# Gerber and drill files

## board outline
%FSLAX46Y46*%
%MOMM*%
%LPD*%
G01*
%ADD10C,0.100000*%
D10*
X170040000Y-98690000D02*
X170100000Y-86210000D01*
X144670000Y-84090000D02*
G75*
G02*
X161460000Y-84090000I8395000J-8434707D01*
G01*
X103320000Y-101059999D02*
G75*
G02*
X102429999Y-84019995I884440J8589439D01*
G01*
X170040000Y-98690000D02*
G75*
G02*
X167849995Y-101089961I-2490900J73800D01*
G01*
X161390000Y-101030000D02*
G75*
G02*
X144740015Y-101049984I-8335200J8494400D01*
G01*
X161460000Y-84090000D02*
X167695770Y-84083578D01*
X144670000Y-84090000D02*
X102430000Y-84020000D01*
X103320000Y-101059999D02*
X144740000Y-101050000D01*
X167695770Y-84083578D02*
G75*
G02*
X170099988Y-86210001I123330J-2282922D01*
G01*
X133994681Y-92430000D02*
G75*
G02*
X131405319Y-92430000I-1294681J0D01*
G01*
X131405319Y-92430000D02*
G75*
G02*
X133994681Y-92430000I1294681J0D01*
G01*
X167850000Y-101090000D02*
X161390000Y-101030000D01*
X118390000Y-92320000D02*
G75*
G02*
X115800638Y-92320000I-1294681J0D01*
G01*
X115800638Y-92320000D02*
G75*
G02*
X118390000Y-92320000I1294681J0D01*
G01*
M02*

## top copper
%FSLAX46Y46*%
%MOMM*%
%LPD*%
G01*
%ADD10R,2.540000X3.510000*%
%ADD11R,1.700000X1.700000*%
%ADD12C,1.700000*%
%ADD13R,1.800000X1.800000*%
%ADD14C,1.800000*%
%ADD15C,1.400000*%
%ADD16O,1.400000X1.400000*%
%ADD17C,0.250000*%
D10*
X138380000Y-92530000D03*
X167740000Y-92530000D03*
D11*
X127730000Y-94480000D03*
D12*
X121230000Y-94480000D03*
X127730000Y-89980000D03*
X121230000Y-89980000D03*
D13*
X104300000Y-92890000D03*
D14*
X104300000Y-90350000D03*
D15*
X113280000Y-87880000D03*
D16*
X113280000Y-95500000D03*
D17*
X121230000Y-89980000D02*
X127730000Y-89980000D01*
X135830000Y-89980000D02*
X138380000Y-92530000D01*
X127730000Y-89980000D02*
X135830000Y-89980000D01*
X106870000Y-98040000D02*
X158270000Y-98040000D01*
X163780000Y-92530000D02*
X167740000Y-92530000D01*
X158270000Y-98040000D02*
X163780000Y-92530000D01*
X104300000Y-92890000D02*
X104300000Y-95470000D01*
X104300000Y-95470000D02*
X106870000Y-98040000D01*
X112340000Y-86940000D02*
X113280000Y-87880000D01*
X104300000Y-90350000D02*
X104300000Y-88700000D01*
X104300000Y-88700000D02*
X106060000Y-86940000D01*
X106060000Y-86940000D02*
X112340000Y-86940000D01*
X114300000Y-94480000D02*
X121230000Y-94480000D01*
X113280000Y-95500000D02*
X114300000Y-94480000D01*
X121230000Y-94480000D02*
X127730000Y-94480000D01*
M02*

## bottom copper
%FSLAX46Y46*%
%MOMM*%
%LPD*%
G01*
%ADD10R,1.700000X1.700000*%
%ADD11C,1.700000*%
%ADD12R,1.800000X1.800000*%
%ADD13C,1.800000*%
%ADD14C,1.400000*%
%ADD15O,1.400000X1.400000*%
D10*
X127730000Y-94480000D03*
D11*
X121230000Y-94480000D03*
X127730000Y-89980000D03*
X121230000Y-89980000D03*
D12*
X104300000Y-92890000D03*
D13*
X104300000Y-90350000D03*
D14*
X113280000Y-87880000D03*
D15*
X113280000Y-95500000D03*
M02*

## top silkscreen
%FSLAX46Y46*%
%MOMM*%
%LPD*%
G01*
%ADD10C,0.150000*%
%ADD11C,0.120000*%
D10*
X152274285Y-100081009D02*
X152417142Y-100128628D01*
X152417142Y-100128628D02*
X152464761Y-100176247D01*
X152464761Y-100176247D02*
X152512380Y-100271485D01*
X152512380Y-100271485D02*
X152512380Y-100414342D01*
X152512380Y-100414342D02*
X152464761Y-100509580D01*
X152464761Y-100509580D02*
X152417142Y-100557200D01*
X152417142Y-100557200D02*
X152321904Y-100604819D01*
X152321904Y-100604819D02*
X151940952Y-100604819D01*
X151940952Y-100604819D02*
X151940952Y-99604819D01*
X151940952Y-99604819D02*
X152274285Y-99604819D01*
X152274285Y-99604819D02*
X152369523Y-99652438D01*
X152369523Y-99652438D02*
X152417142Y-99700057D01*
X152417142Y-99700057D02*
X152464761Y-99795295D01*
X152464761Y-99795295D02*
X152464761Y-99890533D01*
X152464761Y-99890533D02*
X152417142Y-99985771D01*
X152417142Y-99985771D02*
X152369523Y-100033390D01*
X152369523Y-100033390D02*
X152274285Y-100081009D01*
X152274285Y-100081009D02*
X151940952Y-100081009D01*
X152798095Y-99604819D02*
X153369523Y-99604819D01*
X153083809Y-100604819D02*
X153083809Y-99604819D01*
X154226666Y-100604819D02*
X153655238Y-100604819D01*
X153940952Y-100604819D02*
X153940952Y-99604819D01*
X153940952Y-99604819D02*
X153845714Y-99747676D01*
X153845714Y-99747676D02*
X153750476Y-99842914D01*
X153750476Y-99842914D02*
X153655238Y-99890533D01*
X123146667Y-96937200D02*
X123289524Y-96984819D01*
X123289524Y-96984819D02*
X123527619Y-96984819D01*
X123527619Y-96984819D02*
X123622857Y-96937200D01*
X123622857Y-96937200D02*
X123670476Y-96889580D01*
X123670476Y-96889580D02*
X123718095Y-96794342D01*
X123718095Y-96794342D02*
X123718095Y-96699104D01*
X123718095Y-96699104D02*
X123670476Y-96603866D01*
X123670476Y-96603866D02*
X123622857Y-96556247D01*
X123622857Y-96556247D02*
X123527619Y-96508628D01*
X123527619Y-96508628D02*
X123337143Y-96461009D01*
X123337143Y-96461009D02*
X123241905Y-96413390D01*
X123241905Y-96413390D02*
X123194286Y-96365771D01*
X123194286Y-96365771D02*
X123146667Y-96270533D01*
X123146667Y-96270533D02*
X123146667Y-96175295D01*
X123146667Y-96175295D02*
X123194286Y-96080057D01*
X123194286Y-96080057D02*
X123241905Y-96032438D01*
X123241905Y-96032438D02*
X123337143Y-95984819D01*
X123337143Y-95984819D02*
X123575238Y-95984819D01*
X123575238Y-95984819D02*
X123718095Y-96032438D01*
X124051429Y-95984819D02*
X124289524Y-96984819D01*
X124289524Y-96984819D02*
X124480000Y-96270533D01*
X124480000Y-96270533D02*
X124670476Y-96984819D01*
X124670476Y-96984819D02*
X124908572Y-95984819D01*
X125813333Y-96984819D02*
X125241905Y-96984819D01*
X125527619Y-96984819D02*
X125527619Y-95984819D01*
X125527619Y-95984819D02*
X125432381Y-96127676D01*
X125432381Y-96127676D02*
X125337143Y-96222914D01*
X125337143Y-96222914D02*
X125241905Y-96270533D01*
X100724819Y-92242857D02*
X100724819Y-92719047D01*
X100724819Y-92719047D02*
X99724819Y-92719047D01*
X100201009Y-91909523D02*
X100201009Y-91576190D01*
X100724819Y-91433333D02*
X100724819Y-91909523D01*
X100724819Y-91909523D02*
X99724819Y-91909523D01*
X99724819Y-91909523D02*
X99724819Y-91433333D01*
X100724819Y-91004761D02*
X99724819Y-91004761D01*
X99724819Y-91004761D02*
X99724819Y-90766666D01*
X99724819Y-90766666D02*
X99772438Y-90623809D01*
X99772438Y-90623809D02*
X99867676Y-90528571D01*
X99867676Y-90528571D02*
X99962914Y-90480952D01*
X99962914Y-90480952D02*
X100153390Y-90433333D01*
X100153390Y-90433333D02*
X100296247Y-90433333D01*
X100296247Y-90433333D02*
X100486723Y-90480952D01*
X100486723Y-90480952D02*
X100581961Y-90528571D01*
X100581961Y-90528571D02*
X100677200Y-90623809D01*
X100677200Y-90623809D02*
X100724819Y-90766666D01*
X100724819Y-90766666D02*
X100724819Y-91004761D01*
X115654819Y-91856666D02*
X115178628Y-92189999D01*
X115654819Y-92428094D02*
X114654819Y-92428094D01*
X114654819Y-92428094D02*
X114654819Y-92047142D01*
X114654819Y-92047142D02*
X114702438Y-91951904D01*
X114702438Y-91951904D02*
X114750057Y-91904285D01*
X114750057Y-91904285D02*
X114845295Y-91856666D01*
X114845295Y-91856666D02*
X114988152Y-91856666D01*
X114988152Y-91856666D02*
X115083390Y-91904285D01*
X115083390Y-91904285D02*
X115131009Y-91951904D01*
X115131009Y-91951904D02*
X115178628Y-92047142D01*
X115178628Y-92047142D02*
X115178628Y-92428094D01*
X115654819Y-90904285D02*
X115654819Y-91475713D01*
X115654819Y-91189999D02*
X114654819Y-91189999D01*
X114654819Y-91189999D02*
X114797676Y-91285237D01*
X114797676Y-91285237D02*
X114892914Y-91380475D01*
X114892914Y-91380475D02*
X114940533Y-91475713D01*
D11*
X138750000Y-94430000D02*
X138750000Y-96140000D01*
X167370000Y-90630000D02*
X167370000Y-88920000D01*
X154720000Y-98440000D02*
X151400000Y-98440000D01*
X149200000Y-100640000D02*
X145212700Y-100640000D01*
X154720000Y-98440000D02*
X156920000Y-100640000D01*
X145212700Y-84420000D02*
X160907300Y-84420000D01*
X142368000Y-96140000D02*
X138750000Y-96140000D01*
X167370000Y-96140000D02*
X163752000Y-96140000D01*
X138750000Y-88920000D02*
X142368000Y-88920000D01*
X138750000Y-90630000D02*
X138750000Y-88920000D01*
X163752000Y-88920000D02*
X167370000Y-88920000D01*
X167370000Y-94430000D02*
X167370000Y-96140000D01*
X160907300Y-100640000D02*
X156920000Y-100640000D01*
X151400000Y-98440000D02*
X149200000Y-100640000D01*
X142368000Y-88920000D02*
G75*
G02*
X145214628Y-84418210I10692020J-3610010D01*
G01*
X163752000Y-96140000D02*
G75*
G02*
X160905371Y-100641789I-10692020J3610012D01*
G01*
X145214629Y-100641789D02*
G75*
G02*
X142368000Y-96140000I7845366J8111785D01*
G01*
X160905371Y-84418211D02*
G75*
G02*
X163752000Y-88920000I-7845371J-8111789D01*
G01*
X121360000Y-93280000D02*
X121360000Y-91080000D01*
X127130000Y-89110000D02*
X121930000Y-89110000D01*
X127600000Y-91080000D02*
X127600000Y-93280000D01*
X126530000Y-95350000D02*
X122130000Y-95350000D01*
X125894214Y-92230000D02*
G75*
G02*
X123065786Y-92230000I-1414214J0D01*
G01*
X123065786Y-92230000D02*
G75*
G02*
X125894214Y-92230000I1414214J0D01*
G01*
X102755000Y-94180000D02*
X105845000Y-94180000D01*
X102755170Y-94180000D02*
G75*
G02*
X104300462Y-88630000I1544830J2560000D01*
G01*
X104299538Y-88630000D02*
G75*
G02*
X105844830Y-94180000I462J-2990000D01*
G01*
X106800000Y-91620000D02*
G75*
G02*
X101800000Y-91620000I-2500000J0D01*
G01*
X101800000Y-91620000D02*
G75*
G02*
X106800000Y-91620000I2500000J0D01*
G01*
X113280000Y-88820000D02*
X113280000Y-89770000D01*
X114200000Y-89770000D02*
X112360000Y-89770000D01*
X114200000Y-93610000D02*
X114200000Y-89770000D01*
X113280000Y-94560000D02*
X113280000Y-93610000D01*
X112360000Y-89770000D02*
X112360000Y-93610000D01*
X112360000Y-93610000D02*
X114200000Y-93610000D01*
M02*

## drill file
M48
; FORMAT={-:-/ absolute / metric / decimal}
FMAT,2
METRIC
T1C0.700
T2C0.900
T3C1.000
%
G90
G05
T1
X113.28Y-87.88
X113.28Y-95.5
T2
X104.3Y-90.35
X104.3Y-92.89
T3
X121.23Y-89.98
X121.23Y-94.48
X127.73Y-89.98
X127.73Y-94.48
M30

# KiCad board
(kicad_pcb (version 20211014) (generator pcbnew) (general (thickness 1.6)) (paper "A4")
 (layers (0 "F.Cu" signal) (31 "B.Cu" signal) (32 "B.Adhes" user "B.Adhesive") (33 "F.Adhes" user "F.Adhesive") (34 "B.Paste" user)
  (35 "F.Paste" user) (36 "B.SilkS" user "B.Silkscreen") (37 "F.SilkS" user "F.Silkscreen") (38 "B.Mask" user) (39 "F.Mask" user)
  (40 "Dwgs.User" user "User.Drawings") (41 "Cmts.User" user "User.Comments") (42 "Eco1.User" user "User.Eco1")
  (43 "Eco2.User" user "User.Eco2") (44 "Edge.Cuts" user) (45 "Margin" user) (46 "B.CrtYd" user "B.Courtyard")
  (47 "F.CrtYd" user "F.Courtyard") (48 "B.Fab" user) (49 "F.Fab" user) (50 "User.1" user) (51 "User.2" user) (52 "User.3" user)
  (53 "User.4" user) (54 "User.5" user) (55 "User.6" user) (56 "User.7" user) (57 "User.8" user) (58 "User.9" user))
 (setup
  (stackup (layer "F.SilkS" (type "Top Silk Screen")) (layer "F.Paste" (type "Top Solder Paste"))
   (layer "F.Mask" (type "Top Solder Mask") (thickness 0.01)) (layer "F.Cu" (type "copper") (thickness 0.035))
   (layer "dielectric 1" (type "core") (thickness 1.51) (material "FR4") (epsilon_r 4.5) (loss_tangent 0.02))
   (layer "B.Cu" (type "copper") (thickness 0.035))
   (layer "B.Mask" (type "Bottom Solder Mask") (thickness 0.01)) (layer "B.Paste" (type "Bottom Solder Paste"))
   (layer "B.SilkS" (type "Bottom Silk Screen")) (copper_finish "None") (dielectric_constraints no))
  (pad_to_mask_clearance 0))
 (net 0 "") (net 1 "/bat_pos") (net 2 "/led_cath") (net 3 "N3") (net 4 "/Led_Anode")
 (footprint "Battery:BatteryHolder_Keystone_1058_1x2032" (layer "F.Cu") (at 153.06 92.53)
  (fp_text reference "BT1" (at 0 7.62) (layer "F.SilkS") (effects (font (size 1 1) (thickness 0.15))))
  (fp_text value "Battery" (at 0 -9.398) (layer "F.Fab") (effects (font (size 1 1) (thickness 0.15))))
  (fp_line (start -14.31 1.9) (end -14.31 3.61) (layer "F.SilkS") (width 0.12))
  (fp_line (start 14.31 -1.9) (end 14.31 -3.61) (layer "F.SilkS") (width 0.12))
  (fp_line (start 1.66 5.91) (end -1.66 5.91) (layer "F.SilkS") (width 0.12))
  (fp_line (start -3.86 8.11) (end -7.8473 8.11) (layer "F.SilkS") (width 0.12))
  (fp_line (start 1.66 5.91) (end 3.86 8.11) (layer "F.SilkS") (width 0.12))
  (fp_line (start -7.8473 -8.11) (end 7.8473 -8.11) (layer "F.SilkS") (width 0.12))
  (fp_line (start -10.692 3.61) (end -14.31 3.61) (layer "F.SilkS") (width 0.12))
  (fp_line (start 14.31 3.61) (end 10.692 3.61) (layer "F.SilkS") (width 0.12))
  (fp_line (start -14.31 -3.61) (end -10.692 -3.61) (layer "F.SilkS") (width 0.12))
  (fp_line (start -14.31 -1.9) (end -14.31 -3.61) (layer "F.SilkS") (width 0.12))
  (fp_line (start 10.692 -3.61) (end 14.31 -3.61) (layer "F.SilkS") (width 0.12))
  (fp_line (start 14.31 1.9) (end 14.31 3.61) (layer "F.SilkS") (width 0.12))
  (fp_line (start 7.8473 8.11) (end 3.86 8.11) (layer "F.SilkS") (width 0.12))
  (fp_line (start -1.66 5.91) (end -3.86 8.11) (layer "F.SilkS") (width 0.12))
  (fp_arc (start -10.692 -3.61) (mid -9.538084 -6.031244) (end -7.845371 -8.111789) (layer "F.SilkS") (width 0.12))
  (fp_arc (start 10.692 3.61) (mid 9.538084 6.031244) (end 7.845371 8.111789) (layer "F.SilkS") (width 0.12))
  (fp_arc (start -7.845371 8.111789) (mid -9.538085 6.031244) (end -10.692 3.61) (layer "F.SilkS") (width 0.12))
  (fp_arc (start 7.845371 -8.111789) (mid 9.538085 -6.031244) (end 10.692 -3.61) (layer "F.SilkS") (width 0.12))
  (pad "1" smd rect (at -14.68 0) (size 2.54 3.51) (layers "F.Cu" "F.Paste" "F.Mask") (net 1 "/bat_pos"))
  (pad "2" smd rect (at 14.68 0) (size 2.54 3.51) (layers "F.Cu" "F.Paste" "F.Mask") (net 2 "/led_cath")))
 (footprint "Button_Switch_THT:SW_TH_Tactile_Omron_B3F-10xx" (layer "F.Cu") (at 127.73 94.48 180)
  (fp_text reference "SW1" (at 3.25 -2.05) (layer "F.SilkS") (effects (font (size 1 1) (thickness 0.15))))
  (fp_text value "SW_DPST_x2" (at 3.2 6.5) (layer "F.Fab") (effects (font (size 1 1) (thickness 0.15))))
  (fp_line (start 6.37 1.2) (end 6.37 3.4) (layer "F.SilkS") (width 0.12))
  (fp_line (start 0.6 5.37) (end 5.8 5.37) (layer "F.SilkS") (width 0.12))
  (fp_line (start 0.13 3.4) (end 0.13 1.2) (layer "F.SilkS") (width 0.12))
  (fp_line (start 1.2 -0.87) (end 5.6 -0.87) (layer "F.SilkS") (width 0.12))
  (fp_circle (center 3.25 2.25) (end 4.25 3.25) (layer "F.SilkS") (width 0.12) (fill none))
  (pad "1" thru_hole rect (at 0 0 180) (size 1.7 1.7) (drill 1) (layers *.Cu *.Mask) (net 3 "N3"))
  (pad "1" thru_hole circle (at 6.5 0 180) (size 1.7 1.7) (drill 1) (layers *.Cu *.Mask) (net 3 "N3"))
  (pad "2" thru_hole circle (at 0 4.5 180) (size 1.7 1.7) (drill 1) (layers *.Cu *.Mask) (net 1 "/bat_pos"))
  (pad "2" thru_hole circle (at 6.5 4.5 180) (size 1.7 1.7) (drill 1) (layers *.Cu *.Mask) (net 1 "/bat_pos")))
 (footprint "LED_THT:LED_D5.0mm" (layer "F.Cu") (at 104.3 92.89 90)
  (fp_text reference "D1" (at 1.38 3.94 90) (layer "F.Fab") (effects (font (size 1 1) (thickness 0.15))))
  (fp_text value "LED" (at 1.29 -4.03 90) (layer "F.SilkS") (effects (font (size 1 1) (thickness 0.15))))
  (fp_line (start -1.29 -1.545) (end -1.29 1.545) (layer "F.SilkS") (width 0.12))
  (fp_arc (start -1.29 -1.54483) (mid 2.072002 -2.880433) (end 4.26 0.000462) (layer "F.SilkS") (width 0.12))
  (fp_arc (start 4.26 -0.000462) (mid 2.072002 2.880433) (end -1.29 1.54483) (layer "F.SilkS") (width 0.12))
  (fp_circle (center 1.27 0) (end 3.77 0) (layer "F.SilkS") (width 0.12) (fill none))
  (pad "1" thru_hole rect (at 0 0 90) (size 1.8 1.8) (drill 0.9) (layers *.Cu *.Mask) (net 2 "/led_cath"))
  (pad "2" thru_hole circle (at 2.54 0 90) (size 1.8 1.8) (drill 0.9) (layers *.Cu *.Mask) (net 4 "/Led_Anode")))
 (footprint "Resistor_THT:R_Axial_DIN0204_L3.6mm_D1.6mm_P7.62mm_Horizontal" (layer "F.Cu") (at 113.28 87.88 -90)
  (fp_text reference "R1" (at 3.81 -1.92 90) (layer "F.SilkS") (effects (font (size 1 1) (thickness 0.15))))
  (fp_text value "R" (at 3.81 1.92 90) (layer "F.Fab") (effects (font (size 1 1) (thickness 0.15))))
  (fp_line (start 0.94 0) (end 1.89 0) (layer "F.SilkS") (width 0.12))
  (fp_line (start 1.89 -0.92) (end 1.89 0.92) (layer "F.SilkS") (width 0.12))
  (fp_line (start 5.73 -0.92) (end 1.89 -0.92) (layer "F.SilkS") (width 0.12))
  (fp_line (start 6.68 0) (end 5.73 0) (layer "F.SilkS") (width 0.12))
  (fp_line (start 1.89 0.92) (end 5.73 0.92) (layer "F.SilkS") (width 0.12))
  (fp_line (start 5.73 0.92) (end 5.73 -0.92) (layer "F.SilkS") (width 0.12))
  (pad "1" thru_hole circle (at 0 0 270) (size 1.4 1.4) (drill 0.7) (layers *.Cu *.Mask) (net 4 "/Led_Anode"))
  (pad "2" thru_hole oval (at 7.62 0 270) (size 1.4 1.4) (drill 0.7) (layers *.Cu *.Mask) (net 3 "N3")))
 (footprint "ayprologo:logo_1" (layer "B.Cu") (at 152.86 91.7 180)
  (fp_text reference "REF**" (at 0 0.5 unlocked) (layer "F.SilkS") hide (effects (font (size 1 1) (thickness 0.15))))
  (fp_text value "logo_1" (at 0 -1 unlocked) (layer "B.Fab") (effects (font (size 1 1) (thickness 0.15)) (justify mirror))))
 (gr_line (start 170.04 98.69) (end 170.1 86.21) (layer "Edge.Cuts") (width 0.1))
 (gr_arc (start 144.67 84.09) (mid 153.065 80.624274) (end 161.46 84.09) (layer "Edge.Cuts") (width 0.1))
 (gr_arc (start 103.32 101.059999) (mid 95.581339 92.920947) (end 102.43 84.02) (layer "Edge.Cuts") (width 0.1))
 (gr_arc (start 170.04 98.69) (mid 169.389899 100.295971) (end 167.85 101.09) (layer "Edge.Cuts") (width 0.1))
 (gr_arc (start 161.39 101.03) (mid 153.06908 104.436459) (end 144.74 101.05) (layer "Edge.Cuts") (width 0.1))
 (gr_line (start 161.46 84.09) (end 167.69577 84.083578) (layer "Edge.Cuts") (width 0.1))
 (gr_line (start 144.67 84.09) (end 102.43 84.02) (layer "Edge.Cuts") (width 0.1))
 (gr_line (start 103.32 101.059999) (end 144.74 101.05) (layer "Edge.Cuts") (width 0.1))
 (gr_arc (start 167.69577 84.083578) (mid 169.33377 84.653958) (end 170.1 86.21) (layer "Edge.Cuts") (width 0.1))
 (gr_circle (center 132.7 92.43) (end 133.99 92.32) (layer "Edge.Cuts") (width 0.1) (fill none))
 (gr_line (start 167.85 101.09) (end 161.39 101.03) (layer "Edge.Cuts") (width 0.1))
 (gr_circle (center 117.095319 92.32) (end 118.385319 92.21) (layer "Edge.Cuts") (width 0.1) (fill none))
 (segment (start 121.23 89.98) (end 127.73 89.98) (width 0.25) (layer "F.Cu") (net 1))
 (segment (start 135.83 89.98) (end 138.38 92.53) (width 0.25) (layer "F.Cu") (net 1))
 (segment (start 127.73 89.98) (end 135.83 89.98) (width 0.25) (layer "F.Cu") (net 1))
 (segment (start 106.87 98.04) (end 158.27 98.04) (width 0.25) (layer "F.Cu") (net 2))
 (segment (start 163.78 92.53) (end 167.74 92.53) (width 0.25) (layer "F.Cu") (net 2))
 (segment (start 158.27 98.04) (end 163.78 92.53) (width 0.25) (layer "F.Cu") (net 2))
 (segment (start 104.3 92.89) (end 104.3 95.47) (width 0.25) (layer "F.Cu") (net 2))
 (segment (start 104.3 95.47) (end 106.87 98.04) (width 0.25) (layer "F.Cu") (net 2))
 (segment (start 112.34 86.94) (end 113.28 87.88) (width 0.25) (layer "F.Cu") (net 4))
 (segment (start 104.3 90.35) (end 104.3 88.7) (width 0.25) (layer "F.Cu") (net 4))
 (segment (start 104.3 88.7) (end 106.06 86.94) (width 0.25) (layer "F.Cu") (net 4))
 (segment (start 106.06 86.94) (end 112.34 86.94) (width 0.25) (layer "F.Cu") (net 4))
 (segment (start 114.3 94.48) (end 121.23 94.48) (width 0.25) (layer "F.Cu") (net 3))
 (segment (start 113.28 95.5) (end 114.3 94.48) (width 0.25) (layer "F.Cu") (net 3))
 (segment (start 121.23 94.48) (end 127.73 94.48) (width 0.25) (layer "F.Cu") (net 3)))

